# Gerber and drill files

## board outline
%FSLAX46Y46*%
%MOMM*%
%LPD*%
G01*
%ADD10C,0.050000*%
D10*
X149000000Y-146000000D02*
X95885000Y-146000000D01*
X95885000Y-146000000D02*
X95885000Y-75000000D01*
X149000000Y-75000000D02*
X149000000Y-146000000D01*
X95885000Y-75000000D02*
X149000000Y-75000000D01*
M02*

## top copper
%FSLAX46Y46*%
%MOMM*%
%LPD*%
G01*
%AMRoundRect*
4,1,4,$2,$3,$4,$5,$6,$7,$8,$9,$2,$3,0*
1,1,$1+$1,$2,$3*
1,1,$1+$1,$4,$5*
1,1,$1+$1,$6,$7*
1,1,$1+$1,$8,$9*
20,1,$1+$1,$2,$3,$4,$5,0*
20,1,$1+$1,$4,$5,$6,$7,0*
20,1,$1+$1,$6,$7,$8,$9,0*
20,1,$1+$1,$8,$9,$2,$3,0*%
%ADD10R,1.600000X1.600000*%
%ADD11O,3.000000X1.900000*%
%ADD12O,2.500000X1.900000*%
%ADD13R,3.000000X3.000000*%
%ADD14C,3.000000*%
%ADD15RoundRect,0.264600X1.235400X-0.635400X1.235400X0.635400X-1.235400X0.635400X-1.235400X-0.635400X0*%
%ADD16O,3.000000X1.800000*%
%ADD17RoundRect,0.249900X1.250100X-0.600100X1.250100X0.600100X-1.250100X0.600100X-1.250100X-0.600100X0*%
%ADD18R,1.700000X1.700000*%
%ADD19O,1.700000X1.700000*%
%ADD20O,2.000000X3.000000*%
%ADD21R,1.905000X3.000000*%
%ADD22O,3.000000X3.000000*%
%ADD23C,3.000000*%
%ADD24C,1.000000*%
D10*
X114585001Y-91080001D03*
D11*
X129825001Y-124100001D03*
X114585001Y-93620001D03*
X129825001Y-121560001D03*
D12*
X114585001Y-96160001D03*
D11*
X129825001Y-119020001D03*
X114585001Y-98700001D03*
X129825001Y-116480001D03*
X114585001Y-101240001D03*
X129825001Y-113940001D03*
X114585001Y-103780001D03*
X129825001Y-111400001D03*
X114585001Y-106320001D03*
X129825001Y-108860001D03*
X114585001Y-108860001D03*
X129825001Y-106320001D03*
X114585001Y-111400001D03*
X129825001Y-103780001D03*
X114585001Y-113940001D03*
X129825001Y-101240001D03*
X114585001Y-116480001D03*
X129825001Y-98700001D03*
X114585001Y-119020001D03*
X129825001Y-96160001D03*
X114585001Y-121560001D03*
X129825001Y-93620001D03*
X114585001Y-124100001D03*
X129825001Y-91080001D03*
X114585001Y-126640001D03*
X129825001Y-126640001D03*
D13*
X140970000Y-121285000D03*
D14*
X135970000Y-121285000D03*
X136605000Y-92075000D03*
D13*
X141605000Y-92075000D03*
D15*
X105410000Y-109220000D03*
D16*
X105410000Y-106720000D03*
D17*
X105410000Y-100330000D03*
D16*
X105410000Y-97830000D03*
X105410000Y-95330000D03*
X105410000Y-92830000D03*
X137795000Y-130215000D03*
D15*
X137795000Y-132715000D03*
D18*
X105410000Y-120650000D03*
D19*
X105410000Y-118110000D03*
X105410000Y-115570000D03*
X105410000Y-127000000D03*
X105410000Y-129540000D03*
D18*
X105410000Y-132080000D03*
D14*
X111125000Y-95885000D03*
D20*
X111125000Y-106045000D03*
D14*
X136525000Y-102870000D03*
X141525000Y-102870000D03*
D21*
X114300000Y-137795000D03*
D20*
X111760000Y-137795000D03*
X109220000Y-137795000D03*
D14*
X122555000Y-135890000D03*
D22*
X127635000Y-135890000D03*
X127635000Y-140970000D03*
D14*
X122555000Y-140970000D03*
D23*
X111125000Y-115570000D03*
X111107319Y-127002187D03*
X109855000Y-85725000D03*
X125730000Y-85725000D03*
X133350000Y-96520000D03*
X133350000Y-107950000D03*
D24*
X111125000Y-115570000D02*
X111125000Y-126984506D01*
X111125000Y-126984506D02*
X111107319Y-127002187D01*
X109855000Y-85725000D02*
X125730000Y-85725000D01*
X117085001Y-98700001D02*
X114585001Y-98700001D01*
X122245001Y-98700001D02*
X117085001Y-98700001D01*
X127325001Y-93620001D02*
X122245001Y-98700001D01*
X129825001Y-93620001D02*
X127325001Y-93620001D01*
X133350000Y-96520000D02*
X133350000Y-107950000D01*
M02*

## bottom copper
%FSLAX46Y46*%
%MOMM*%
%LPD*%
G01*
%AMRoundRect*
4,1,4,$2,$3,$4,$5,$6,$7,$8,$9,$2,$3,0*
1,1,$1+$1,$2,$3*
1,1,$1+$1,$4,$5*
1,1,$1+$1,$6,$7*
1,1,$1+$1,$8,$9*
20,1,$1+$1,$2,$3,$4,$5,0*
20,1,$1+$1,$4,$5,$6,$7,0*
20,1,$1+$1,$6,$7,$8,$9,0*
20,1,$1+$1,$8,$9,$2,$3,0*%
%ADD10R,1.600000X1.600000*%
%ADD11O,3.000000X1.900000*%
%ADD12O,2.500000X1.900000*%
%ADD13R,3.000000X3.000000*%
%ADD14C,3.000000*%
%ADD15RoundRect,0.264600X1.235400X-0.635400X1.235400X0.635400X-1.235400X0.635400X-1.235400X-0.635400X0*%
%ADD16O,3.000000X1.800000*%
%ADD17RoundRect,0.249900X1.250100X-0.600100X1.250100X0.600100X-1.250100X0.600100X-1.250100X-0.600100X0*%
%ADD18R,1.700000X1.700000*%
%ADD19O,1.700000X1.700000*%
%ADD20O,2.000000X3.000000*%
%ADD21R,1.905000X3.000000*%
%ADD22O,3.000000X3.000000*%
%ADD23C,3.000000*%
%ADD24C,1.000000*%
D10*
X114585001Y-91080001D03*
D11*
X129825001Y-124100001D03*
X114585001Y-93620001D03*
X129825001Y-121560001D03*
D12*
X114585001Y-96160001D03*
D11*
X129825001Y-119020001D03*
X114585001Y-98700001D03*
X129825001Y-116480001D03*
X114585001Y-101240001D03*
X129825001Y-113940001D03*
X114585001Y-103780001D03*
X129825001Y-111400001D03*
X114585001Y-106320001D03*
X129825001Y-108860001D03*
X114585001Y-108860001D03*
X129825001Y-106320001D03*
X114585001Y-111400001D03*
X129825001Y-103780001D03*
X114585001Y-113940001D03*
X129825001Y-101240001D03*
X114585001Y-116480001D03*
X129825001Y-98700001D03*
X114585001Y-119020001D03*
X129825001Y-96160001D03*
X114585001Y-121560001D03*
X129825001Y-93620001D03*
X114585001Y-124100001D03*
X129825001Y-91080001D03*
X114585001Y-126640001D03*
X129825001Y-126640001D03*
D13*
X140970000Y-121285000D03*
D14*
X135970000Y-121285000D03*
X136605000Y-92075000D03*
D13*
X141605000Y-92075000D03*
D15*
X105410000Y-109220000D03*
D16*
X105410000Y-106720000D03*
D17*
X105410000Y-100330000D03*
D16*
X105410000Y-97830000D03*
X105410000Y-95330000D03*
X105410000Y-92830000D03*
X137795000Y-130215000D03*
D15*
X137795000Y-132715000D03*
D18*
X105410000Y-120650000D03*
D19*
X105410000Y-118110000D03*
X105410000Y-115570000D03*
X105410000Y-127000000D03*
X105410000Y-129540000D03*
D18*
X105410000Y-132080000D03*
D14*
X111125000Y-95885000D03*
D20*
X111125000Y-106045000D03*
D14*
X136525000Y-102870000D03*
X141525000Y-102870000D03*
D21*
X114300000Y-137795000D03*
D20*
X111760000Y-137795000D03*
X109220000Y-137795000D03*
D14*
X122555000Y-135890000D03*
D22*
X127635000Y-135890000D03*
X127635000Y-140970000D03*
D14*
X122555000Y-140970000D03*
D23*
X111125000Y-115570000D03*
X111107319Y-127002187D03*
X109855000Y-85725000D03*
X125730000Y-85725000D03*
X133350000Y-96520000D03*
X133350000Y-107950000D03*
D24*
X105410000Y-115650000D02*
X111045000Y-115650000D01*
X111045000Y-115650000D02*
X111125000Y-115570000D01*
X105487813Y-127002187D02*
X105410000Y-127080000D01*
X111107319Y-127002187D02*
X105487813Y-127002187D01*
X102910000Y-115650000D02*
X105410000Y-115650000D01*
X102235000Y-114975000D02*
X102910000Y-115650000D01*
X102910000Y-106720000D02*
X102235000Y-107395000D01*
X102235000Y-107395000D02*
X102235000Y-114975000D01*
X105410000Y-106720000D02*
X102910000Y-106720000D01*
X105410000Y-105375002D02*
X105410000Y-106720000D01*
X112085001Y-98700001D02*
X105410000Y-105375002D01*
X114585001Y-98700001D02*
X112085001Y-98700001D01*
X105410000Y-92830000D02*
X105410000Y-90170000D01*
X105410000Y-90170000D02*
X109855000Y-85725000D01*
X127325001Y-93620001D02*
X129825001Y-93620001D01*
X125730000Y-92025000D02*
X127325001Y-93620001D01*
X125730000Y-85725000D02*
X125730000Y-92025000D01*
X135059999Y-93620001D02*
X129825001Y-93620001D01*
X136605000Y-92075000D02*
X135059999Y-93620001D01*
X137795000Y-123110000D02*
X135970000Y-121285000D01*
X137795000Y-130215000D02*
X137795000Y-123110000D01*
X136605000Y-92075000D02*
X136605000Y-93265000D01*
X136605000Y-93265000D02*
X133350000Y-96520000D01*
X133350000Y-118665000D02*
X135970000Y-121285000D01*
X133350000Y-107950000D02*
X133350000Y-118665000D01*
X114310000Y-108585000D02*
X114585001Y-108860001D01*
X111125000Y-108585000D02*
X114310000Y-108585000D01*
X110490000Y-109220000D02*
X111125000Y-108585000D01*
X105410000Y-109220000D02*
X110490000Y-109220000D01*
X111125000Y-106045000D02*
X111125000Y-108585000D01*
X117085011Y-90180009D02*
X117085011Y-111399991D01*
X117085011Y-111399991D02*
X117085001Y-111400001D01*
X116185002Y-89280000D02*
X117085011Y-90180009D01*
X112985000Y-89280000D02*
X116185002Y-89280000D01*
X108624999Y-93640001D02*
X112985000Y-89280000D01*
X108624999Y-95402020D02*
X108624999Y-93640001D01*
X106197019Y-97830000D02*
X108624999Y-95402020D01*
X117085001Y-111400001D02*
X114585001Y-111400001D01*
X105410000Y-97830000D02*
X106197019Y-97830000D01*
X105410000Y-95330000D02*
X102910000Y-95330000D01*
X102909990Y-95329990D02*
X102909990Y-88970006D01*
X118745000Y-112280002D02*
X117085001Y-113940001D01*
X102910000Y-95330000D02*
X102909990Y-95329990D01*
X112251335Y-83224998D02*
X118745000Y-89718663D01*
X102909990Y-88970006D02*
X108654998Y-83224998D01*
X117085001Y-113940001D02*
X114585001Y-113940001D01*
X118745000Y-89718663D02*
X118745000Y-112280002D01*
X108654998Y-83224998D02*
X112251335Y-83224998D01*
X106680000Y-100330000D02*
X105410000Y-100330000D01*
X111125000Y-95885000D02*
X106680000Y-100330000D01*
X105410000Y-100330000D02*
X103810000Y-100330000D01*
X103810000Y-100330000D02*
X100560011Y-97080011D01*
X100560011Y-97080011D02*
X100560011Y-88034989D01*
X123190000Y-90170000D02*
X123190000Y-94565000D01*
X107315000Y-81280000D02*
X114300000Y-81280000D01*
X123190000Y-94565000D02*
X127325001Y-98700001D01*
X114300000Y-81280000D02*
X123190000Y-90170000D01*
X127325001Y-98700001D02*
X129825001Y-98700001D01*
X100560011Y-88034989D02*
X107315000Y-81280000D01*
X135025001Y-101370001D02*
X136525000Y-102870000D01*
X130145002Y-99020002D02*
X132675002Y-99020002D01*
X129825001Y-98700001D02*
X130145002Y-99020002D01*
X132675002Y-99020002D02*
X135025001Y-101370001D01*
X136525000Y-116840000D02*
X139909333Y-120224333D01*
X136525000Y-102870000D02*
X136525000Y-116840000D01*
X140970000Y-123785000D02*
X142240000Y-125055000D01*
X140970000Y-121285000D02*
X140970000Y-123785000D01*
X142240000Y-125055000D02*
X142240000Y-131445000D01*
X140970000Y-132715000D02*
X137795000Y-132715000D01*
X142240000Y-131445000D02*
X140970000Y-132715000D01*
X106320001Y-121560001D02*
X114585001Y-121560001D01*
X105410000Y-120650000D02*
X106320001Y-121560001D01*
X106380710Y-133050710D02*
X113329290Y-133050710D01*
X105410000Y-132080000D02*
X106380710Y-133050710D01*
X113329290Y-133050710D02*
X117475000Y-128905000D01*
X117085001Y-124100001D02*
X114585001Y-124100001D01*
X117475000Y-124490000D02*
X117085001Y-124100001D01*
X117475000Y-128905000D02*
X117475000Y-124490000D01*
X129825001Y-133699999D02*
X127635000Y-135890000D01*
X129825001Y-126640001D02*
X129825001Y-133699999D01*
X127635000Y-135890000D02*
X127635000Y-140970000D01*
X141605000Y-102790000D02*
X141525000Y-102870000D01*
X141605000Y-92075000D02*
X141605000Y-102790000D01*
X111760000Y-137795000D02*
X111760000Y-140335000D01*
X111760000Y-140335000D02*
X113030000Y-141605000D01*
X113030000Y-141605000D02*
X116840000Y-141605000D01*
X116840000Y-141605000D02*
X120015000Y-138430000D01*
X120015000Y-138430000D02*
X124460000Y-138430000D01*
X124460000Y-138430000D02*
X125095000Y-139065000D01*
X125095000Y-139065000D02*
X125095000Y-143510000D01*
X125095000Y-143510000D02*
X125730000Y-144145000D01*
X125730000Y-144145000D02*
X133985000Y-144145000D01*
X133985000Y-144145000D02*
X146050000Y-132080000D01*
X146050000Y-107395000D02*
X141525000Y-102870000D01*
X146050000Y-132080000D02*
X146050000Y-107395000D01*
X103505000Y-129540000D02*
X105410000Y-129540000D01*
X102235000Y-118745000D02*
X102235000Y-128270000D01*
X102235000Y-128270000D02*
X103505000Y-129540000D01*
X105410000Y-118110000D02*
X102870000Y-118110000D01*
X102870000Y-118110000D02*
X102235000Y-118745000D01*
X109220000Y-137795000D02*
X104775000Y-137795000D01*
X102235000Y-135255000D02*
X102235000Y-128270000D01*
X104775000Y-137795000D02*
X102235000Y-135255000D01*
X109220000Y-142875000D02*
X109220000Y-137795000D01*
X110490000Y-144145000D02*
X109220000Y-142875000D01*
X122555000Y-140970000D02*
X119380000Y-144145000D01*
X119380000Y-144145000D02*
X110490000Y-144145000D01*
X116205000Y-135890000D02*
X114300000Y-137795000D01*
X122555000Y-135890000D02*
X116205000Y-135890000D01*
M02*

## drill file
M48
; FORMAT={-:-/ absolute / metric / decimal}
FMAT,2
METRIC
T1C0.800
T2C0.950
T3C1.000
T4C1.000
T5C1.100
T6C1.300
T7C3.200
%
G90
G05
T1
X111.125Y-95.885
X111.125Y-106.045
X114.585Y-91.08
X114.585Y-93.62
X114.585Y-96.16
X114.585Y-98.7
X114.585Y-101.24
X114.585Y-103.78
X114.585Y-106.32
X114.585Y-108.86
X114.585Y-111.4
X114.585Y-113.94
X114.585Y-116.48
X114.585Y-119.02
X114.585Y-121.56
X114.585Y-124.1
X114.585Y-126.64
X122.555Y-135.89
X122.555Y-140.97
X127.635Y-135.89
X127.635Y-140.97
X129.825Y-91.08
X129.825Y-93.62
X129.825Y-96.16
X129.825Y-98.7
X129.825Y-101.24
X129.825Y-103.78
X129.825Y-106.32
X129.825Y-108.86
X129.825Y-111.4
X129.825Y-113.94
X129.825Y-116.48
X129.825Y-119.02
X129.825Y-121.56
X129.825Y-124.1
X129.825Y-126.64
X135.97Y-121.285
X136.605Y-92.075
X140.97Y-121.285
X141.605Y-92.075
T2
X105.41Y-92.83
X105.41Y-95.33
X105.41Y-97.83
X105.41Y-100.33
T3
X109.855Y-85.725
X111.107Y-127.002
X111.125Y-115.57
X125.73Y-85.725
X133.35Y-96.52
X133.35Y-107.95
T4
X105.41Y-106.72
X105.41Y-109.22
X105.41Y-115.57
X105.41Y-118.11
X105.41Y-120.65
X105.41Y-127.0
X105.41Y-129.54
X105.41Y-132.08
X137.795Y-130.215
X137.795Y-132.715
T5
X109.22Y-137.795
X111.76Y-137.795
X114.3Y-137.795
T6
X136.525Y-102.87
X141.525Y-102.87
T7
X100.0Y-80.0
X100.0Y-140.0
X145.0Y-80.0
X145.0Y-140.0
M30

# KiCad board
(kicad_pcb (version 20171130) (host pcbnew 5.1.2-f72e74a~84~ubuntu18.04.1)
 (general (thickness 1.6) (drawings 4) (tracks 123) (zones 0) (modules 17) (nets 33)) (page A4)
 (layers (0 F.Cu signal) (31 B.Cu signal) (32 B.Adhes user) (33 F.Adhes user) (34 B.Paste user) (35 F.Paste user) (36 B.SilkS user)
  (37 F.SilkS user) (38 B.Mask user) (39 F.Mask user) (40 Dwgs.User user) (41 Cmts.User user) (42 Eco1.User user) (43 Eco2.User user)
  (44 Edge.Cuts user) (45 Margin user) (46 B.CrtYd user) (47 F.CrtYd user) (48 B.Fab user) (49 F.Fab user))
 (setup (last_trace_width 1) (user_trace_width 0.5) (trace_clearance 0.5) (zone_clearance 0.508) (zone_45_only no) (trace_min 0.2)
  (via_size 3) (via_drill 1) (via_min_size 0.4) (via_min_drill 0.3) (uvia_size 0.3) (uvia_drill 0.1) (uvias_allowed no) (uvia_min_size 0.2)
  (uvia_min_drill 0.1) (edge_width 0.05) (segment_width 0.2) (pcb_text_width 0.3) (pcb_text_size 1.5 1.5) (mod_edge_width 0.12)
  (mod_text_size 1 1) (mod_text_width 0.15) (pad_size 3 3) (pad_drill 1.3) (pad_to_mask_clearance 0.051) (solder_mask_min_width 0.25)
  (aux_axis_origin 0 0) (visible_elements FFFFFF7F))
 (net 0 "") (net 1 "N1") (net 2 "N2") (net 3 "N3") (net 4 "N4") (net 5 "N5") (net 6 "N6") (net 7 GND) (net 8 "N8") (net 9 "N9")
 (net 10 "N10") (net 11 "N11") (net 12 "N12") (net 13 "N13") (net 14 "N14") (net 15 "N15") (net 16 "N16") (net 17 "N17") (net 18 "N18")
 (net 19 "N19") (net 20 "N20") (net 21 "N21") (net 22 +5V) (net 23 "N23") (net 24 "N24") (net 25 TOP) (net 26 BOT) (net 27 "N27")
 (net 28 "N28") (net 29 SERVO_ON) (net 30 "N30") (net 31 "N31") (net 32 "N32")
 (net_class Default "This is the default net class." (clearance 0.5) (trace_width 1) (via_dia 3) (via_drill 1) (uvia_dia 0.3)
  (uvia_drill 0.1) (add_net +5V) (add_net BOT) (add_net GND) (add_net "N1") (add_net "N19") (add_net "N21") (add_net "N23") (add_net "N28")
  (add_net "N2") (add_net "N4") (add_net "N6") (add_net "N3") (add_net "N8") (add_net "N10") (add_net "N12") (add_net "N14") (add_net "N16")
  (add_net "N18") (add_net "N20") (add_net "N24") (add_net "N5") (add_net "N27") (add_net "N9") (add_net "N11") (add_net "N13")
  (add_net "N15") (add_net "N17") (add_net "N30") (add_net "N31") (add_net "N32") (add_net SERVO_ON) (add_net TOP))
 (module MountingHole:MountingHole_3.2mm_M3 (layer F.Cu) (at 145 140)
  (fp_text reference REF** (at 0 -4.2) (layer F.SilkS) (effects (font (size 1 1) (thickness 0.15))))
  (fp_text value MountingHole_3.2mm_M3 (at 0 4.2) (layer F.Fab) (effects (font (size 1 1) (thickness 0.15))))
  (pad 1 np_thru_hole circle (at 0 0) (size 3.2 3.2) (drill 3.2) (layers *.Cu *.Mask)))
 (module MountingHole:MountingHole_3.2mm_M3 (layer F.Cu) (at 100 140)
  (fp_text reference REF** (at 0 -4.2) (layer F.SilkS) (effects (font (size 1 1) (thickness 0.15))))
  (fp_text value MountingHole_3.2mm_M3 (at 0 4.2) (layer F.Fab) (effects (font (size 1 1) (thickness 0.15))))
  (pad 1 np_thru_hole circle (at 0 0) (size 3.2 3.2) (drill 3.2) (layers *.Cu *.Mask)))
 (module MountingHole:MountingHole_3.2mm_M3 (layer F.Cu) (at 100 80)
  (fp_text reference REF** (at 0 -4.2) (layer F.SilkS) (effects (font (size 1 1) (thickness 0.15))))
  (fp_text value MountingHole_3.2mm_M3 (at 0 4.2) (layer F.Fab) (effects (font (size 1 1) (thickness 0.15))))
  (pad 1 np_thru_hole circle (at 0 0) (size 3.2 3.2) (drill 3.2) (layers *.Cu *.Mask)))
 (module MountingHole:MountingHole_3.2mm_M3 (layer F.Cu) (at 145 80)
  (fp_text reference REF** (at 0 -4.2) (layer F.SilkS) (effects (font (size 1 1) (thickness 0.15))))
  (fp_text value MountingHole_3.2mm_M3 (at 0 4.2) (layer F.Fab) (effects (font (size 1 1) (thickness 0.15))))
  (pad 1 np_thru_hole circle (at 0 0) (size 3.2 3.2) (drill 3.2) (layers *.Cu *.Mask)))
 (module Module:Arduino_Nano (layer F.Cu) (at 114.585001 91.080001)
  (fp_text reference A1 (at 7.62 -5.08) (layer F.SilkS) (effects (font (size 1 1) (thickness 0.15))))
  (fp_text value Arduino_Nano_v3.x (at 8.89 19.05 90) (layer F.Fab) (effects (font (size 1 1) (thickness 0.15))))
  (pad 1 thru_hole rect (at 0 0) (size 1.6 1.6) (drill 0.8) (layers *.Cu *.Mask) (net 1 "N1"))
  (pad 17 thru_hole oval (at 15.24 33.02) (size 3 1.9) (drill 0.8) (layers *.Cu *.Mask) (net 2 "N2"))
  (pad 2 thru_hole oval (at 0 2.54) (size 3 1.9) (drill 0.8) (layers *.Cu *.Mask) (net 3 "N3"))
  (pad 18 thru_hole oval (at 15.24 30.48) (size 3 1.9) (drill 0.8) (layers *.Cu *.Mask) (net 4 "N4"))
  (pad 3 thru_hole oval (at 0 5.08) (size 2.5 1.9) (drill 0.8) (layers *.Cu *.Mask) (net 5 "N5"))
  (pad 19 thru_hole oval (at 15.24 27.94) (size 3 1.9) (drill 0.8) (layers *.Cu *.Mask) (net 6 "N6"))
  (pad 4 thru_hole oval (at 0 7.62) (size 3 1.9) (drill 0.8) (layers *.Cu *.Mask) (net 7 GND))
  (pad 20 thru_hole oval (at 15.24 25.4) (size 3 1.9) (drill 0.8) (layers *.Cu *.Mask) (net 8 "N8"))
  (pad 5 thru_hole oval (at 0 10.16) (size 3 1.9) (drill 0.8) (layers *.Cu *.Mask) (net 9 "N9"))
  (pad 21 thru_hole oval (at 15.24 22.86) (size 3 1.9) (drill 0.8) (layers *.Cu *.Mask) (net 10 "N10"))
  (pad 6 thru_hole oval (at 0 12.7) (size 3 1.9) (drill 0.8) (layers *.Cu *.Mask) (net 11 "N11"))
  (pad 22 thru_hole oval (at 15.24 20.32) (size 3 1.9) (drill 0.8) (layers *.Cu *.Mask) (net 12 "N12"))
  (pad 7 thru_hole oval (at 0 15.24) (size 3 1.9) (drill 0.8) (layers *.Cu *.Mask) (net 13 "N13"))
  (pad 23 thru_hole oval (at 15.24 17.78) (size 3 1.9) (drill 0.8) (layers *.Cu *.Mask) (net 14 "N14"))
  (pad 8 thru_hole oval (at 0 17.78) (size 3 1.9) (drill 0.8) (layers *.Cu *.Mask) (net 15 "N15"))
  (pad 24 thru_hole oval (at 15.24 15.24) (size 3 1.9) (drill 0.8) (layers *.Cu *.Mask) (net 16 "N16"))
  (pad 9 thru_hole oval (at 0 20.32) (size 3 1.9) (drill 0.8) (layers *.Cu *.Mask) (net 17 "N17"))
  (pad 25 thru_hole oval (at 15.24 12.7) (size 3 1.9) (drill 0.8) (layers *.Cu *.Mask) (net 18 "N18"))
  (pad 10 thru_hole oval (at 0 22.86) (size 3 1.9) (drill 0.8) (layers *.Cu *.Mask) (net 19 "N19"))
  (pad 26 thru_hole oval (at 15.24 10.16) (size 3 1.9) (drill 0.8) (layers *.Cu *.Mask) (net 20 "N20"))
  (pad 11 thru_hole oval (at 0 25.4) (size 3 1.9) (drill 0.8) (layers *.Cu *.Mask) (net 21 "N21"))
  (pad 27 thru_hole oval (at 15.24 7.62) (size 3 1.9) (drill 0.8) (layers *.Cu *.Mask) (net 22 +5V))
  (pad 12 thru_hole oval (at 0 27.94) (size 3 1.9) (drill 0.8) (layers *.Cu *.Mask) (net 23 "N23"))
  (pad 28 thru_hole oval (at 15.24 5.08) (size 3 1.9) (drill 0.8) (layers *.Cu *.Mask) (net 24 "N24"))
  (pad 13 thru_hole oval (at 0 30.48) (size 3 1.9) (drill 0.8) (layers *.Cu *.Mask) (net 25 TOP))
  (pad 29 thru_hole oval (at 15.24 2.54) (size 3 1.9) (drill 0.8) (layers *.Cu *.Mask) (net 7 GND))
  (pad 14 thru_hole oval (at 0 33.02) (size 3 1.9) (drill 0.8) (layers *.Cu *.Mask) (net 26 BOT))
  (pad 30 thru_hole oval (at 15.24 0) (size 3 1.9) (drill 0.8) (layers *.Cu *.Mask) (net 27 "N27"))
  (pad 15 thru_hole oval (at 0 35.56) (size 3 1.9) (drill 0.8) (layers *.Cu *.Mask) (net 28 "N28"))
  (pad 16 thru_hole oval (at 15.24 35.56) (size 3 1.9) (drill 0.8) (layers *.Cu *.Mask) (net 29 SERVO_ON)))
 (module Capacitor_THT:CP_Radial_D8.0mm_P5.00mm (layer F.Cu) (at 140.97 121.285 180)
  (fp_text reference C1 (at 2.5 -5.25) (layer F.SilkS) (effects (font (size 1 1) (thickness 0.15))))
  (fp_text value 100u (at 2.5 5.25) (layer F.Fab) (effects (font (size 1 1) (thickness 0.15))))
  (pad 1 thru_hole rect (at 0 0 180) (size 3 3) (drill 0.8) (layers *.Cu *.Mask) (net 22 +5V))
  (pad 2 thru_hole circle (at 5 0 180) (size 3 3) (drill 0.8) (layers *.Cu *.Mask) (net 7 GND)))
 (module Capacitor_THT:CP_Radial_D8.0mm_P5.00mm (layer F.Cu) (at 141.605 92.075 180)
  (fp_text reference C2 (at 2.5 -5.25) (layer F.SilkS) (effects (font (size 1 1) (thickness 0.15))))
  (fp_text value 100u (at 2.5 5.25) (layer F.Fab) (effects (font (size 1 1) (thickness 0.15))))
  (pad 2 thru_hole circle (at 5 0 180) (size 3 3) (drill 0.8) (layers *.Cu *.Mask) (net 7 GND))
  (pad 1 thru_hole rect (at 0 0 180) (size 3 3) (drill 0.8) (layers *.Cu *.Mask) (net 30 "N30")))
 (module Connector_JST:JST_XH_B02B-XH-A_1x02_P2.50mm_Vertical (layer F.Cu) (at 105.41 109.22 90)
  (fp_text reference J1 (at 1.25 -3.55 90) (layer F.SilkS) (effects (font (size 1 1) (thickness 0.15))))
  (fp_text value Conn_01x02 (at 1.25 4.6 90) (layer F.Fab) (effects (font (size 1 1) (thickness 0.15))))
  (pad 1 thru_hole roundrect (at 0 0 90) (size 1.8 3) (drill 1) (layers *.Cu *.Mask) (roundrect_rratio 0.147) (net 15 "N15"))
  (pad 2 thru_hole oval (at 2.5 0 90) (size 1.8 3) (drill 1) (layers *.Cu *.Mask) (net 7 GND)))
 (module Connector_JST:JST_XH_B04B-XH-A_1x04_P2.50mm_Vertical (layer F.Cu) (at 105.41 100.33 90)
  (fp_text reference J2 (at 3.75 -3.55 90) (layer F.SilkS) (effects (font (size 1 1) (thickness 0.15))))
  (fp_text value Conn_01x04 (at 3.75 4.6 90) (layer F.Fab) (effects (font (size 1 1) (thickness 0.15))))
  (pad 1 thru_hole roundrect (at 0 0 90) (size 1.7 3) (drill 0.95) (layers *.Cu *.Mask) (roundrect_rratio 0.147) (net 22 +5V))
  (pad 2 thru_hole oval (at 2.5 0 90) (size 1.8 3) (drill 0.95) (layers *.Cu *.Mask) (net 17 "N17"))
  (pad 3 thru_hole oval (at 5 0 90) (size 1.8 3) (drill 0.95) (layers *.Cu *.Mask) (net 19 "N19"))
  (pad 4 thru_hole oval (at 7.5 0 90) (size 1.8 3) (drill 0.95) (layers *.Cu *.Mask) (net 7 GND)))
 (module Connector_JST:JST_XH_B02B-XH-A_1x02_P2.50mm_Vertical (layer F.Cu) (at 137.795 132.715 90)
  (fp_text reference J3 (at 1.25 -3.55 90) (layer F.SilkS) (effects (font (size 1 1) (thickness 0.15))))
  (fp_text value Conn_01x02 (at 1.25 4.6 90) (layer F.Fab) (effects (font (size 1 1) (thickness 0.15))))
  (pad 2 thru_hole oval (at 2.5 0 90) (size 1.8 3) (drill 1) (layers *.Cu *.Mask) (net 7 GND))
  (pad 1 thru_hole roundrect (at 0 0 90) (size 1.8 3) (drill 1) (layers *.Cu *.Mask) (roundrect_rratio 0.147) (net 22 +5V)))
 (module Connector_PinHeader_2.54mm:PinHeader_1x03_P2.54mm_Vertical (layer F.Cu) (at 105.41 120.65 180)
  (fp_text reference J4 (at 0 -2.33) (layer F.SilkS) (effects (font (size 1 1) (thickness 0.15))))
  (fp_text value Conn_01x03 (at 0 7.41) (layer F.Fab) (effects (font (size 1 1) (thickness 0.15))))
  (pad 1 thru_hole rect (at 0 0 180) (size 1.7 1.7) (drill 1) (layers *.Cu *.Mask) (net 25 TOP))
  (pad 2 thru_hole oval (at 0 2.54 180) (size 1.7 1.7) (drill 1) (layers *.Cu *.Mask) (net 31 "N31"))
  (pad 3 thru_hole oval (at 0 5.08 180) (size 1.7 1.7) (drill 1) (layers *.Cu *.Mask) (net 7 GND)))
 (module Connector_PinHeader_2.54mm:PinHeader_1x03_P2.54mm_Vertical (layer F.Cu) (at 105.41 132.08 180)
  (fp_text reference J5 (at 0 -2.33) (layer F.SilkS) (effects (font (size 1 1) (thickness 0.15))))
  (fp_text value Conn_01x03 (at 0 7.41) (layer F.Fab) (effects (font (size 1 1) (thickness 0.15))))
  (pad 3 thru_hole oval (at 0 5.08 180) (size 1.7 1.7) (drill 1) (layers *.Cu *.Mask) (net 7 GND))
  (pad 2 thru_hole oval (at 0 2.54 180) (size 1.7 1.7) (drill 1) (layers *.Cu *.Mask) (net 31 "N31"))
  (pad 1 thru_hole rect (at 0 0 180) (size 1.7 1.7) (drill 1) (layers *.Cu *.Mask) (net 26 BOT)))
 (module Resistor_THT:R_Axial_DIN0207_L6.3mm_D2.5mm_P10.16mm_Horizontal (layer F.Cu) (at 111.125 95.885 270)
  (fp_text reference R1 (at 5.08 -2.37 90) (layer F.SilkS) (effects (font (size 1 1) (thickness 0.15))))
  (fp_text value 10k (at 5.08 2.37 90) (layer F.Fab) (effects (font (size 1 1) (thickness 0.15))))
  (pad 1 thru_hole circle (at 0 0 270) (size 3 3) (drill 0.8) (layers *.Cu *.Mask) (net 22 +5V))
  (pad 2 thru_hole oval (at 10.16 0 270) (size 3 2) (drill 0.8) (layers *.Cu *.Mask) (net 15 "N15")))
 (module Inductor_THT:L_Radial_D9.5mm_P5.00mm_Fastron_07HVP (layer F.Cu) (at 136.525 102.87)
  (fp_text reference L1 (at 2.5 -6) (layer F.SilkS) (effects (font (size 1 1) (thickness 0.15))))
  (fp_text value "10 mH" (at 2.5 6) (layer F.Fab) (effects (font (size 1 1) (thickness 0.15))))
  (pad 1 thru_hole circle (at 0 0) (size 3 3) (drill 1.3) (layers *.Cu *.Mask) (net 22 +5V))
  (pad 2 thru_hole circle (at 5 0) (size 3 3) (drill 1.3) (layers *.Cu *.Mask) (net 30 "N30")))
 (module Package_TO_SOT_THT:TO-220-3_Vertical (layer F.Cu) (at 114.3 137.795 180)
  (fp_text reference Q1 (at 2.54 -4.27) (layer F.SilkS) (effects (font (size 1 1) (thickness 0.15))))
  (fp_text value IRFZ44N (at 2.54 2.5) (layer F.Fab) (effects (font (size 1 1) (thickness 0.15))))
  (pad 1 thru_hole rect (at 0 0 180) (size 1.905 3) (drill 1.1) (layers *.Cu *.Mask) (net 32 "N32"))
  (pad 2 thru_hole oval (at 2.54 0 180) (size 2 3) (drill 1.1) (layers *.Cu *.Mask) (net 30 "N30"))
  (pad 3 thru_hole oval (at 5.08 0 180) (size 2 3) (drill 1.1) (layers *.Cu *.Mask) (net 31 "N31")))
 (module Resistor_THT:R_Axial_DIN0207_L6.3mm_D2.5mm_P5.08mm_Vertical (layer F.Cu) (at 122.555 135.89)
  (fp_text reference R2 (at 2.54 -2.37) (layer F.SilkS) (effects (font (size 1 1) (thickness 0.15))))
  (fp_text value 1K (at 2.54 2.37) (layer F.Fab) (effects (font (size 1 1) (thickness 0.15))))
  (pad 1 thru_hole circle (at 0 0) (size 3 3) (drill 0.8) (layers *.Cu *.Mask) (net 32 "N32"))
  (pad 2 thru_hole oval (at 5.08 0) (size 3 3) (drill 0.8) (layers *.Cu *.Mask) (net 29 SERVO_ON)))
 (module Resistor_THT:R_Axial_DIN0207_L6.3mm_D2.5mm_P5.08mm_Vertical (layer F.Cu) (at 122.555 140.97)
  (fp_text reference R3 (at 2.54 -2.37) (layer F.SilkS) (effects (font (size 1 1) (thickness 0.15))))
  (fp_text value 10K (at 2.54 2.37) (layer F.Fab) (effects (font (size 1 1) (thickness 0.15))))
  (pad 2 thru_hole oval (at 5.08 0) (size 3 3) (drill 0.8) (layers *.Cu *.Mask) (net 29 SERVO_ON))
  (pad 1 thru_hole circle (at 0 0) (size 3 3) (drill 0.8) (layers *.Cu *.Mask) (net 31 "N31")))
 (gr_line (start 149 146) (end 95.885 146) (layer Edge.Cuts) (width 0.05))
 (gr_line (start 95.885 146) (end 95.885 75) (layer Edge.Cuts) (width 0.05))
 (gr_line (start 149 75) (end 149 146) (layer Edge.Cuts) (width 0.05))
 (gr_line (start 95.885 75) (end 149 75) (layer Edge.Cuts) (width 0.05))
 (segment (start 105.41 115.65) (end 111.045 115.65) (width 1) (layer B.Cu) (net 7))
 (via (at 111.125 115.57) (size 3) (drill 1) (layers F.Cu B.Cu) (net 7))
 (segment (start 111.045 115.65) (end 111.125 115.57) (width 1) (layer B.Cu) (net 7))
 (via (at 111.107319 127.002187) (size 3) (drill 1) (layers F.Cu B.Cu) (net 7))
 (segment (start 111.125 115.57) (end 111.125 126.984506) (width 1) (layer F.Cu) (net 7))
 (segment (start 111.125 126.984506) (end 111.107319 127.002187) (width 1) (layer F.Cu) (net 7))
 (segment (start 105.487813 127.002187) (end 105.41 127.08) (width 1) (layer B.Cu) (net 7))
 (segment (start 111.107319 127.002187) (end 105.487813 127.002187) (width 1) (layer B.Cu) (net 7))
 (segment (start 102.91 115.65) (end 105.41 115.65) (width 1) (layer B.Cu) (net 7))
 (segment (start 102.235 114.975) (end 102.91 115.65) (width 1) (layer B.Cu) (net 7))
 (segment (start 102.91 106.72) (end 102.235 107.395) (width 1) (layer B.Cu) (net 7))
 (segment (start 102.235 107.395) (end 102.235 114.975) (width 1) (layer B.Cu) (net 7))
 (segment (start 105.41 106.72) (end 102.91 106.72) (width 1) (layer B.Cu) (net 7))
 (segment (start 105.41 105.375002) (end 105.41 106.72) (width 1) (layer B.Cu) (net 7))
 (segment (start 112.085001 98.700001) (end 105.41 105.375002) (width 1) (layer B.Cu) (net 7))
 (segment (start 114.585001 98.700001) (end 112.085001 98.700001) (width 1) (layer B.Cu) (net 7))
 (segment (start 105.41 92.83) (end 105.41 90.17) (width 1) (layer B.Cu) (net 7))
 (segment (start 105.41 90.17) (end 109.855 85.725) (width 1) (layer B.Cu) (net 7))
 (via (at 109.855 85.725) (size 3) (drill 1) (layers F.Cu B.Cu) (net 7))
 (via (at 125.73 85.725) (size 3) (drill 1) (layers F.Cu B.Cu) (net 7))
 (segment (start 109.855 85.725) (end 125.73 85.725) (width 1) (layer F.Cu) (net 7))
 (segment (start 127.325001 93.620001) (end 129.825001 93.620001) (width 1) (layer B.Cu) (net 7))
 (segment (start 125.73 92.025) (end 127.325001 93.620001) (width 1) (layer B.Cu) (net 7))
 (segment (start 125.73 85.725) (end 125.73 92.025) (width 1) (layer B.Cu) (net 7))
 (segment (start 117.085001 98.700001) (end 114.585001 98.700001) (width 1) (layer F.Cu) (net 7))
 (segment (start 122.245001 98.700001) (end 117.085001 98.700001) (width 1) (layer F.Cu) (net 7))
 (segment (start 127.325001 93.620001) (end 122.245001 98.700001) (width 1) (layer F.Cu) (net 7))
 (segment (start 129.825001 93.620001) (end 127.325001 93.620001) (width 1) (layer F.Cu) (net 7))
 (segment (start 135.059999 93.620001) (end 129.825001 93.620001) (width 1) (layer B.Cu) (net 7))
 (segment (start 136.605 92.075) (end 135.059999 93.620001) (width 1) (layer B.Cu) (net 7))
 (segment (start 137.795 123.11) (end 135.97 121.285) (width 1) (layer B.Cu) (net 7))
 (segment (start 137.795 130.215) (end 137.795 123.11) (width 1) (layer B.Cu) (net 7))
 (via (at 133.35 96.52) (size 3) (drill 1) (layers F.Cu B.Cu) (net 7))
 (segment (start 136.605 92.075) (end 136.605 93.265) (width 1) (layer B.Cu) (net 7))
 (segment (start 136.605 93.265) (end 133.35 96.52) (width 1) (layer B.Cu) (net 7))
 (via (at 133.35 107.95) (size 3) (drill 1) (layers F.Cu B.Cu) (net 7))
 (segment (start 133.35 96.52) (end 133.35 107.95) (width 1) (layer F.Cu) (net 7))
 (segment (start 133.35 118.665) (end 135.97 121.285) (width 1) (layer B.Cu) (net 7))
 (segment (start 133.35 107.95) (end 133.35 118.665) (width 1) (layer B.Cu) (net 7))
 (segment (start 114.31 108.585) (end 114.585001 108.860001) (width 1) (layer B.Cu) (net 15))
 (segment (start 111.125 108.585) (end 114.31 108.585) (width 1) (layer B.Cu) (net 15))
 (segment (start 110.49 109.22) (end 111.125 108.585) (width 1) (layer B.Cu) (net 15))
 (segment (start 105.41 109.22) (end 110.49 109.22) (width 1) (layer B.Cu) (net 15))
 (segment (start 111.125 106.045) (end 111.125 108.585) (width 1) (layer B.Cu) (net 15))
 (segment (start 117.085011 90.180009) (end 117.085011 111.399991) (width 1) (layer B.Cu) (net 17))
 (segment (start 117.085011 111.399991) (end 117.085001 111.400001) (width 1) (layer B.Cu) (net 17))
 (segment (start 116.185002 89.28) (end 117.085011 90.180009) (width 1) (layer B.Cu) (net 17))
 (segment (start 112.985 89.28) (end 116.185002 89.28) (width 1) (layer B.Cu) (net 17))
 (segment (start 108.624999 93.640001) (end 112.985 89.28) (width 1) (layer B.Cu) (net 17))
 (segment (start 108.624999 95.40202) (end 108.624999 93.640001) (width 1) (layer B.Cu) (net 17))
 (segment (start 106.197019 97.83) (end 108.624999 95.40202) (width 1) (layer B.Cu) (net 17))
 (segment (start 117.085001 111.400001) (end 114.585001 111.400001) (width 1) (layer B.Cu) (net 17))
 (segment (start 105.41 97.83) (end 106.197019 97.83) (width 1) (layer B.Cu) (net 17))
 (segment (start 105.41 95.33) (end 102.91 95.33) (width 1) (layer B.Cu) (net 19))
 (segment (start 102.90999 95.32999) (end 102.90999 88.970006) (width 1) (layer B.Cu) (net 19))
 (segment (start 118.745 112.280002) (end 117.085001 113.940001) (width 1) (layer B.Cu) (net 19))
 (segment (start 102.91 95.33) (end 102.90999 95.32999) (width 1) (layer B.Cu) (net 19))
 (segment (start 112.251335 83.224998) (end 118.745 89.718663) (width 1) (layer B.Cu) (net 19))
 (segment (start 102.90999 88.970006) (end 108.654998 83.224998) (width 1) (layer B.Cu) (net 19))
 (segment (start 117.085001 113.940001) (end 114.585001 113.940001) (width 1) (layer B.Cu) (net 19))
 (segment (start 118.745 89.718663) (end 118.745 112.280002) (width 1) (layer B.Cu) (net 19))
 (segment (start 108.654998 83.224998) (end 112.251335 83.224998) (width 1) (layer B.Cu) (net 19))
 (segment (start 106.68 100.33) (end 105.41 100.33) (width 1) (layer B.Cu) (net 22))
 (segment (start 111.125 95.885) (end 106.68 100.33) (width 1) (layer B.Cu) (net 22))
 (segment (start 105.41 100.33) (end 103.81 100.33) (width 1) (layer B.Cu) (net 22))
 (segment (start 103.81 100.33) (end 100.560011 97.080011) (width 1) (layer B.Cu) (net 22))
 (segment (start 100.560011 97.080011) (end 100.560011 88.034989) (width 1) (layer B.Cu) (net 22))
 (segment (start 123.19 90.17) (end 123.19 94.565) (width 1) (layer B.Cu) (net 22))
 (segment (start 107.315 81.28) (end 114.3 81.28) (width 1) (layer B.Cu) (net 22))
 (segment (start 123.19 94.565) (end 127.325001 98.700001) (width 1) (layer B.Cu) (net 22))
 (segment (start 114.3 81.28) (end 123.19 90.17) (width 1) (layer B.Cu) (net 22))
 (segment (start 127.325001 98.700001) (end 129.825001 98.700001) (width 1) (layer B.Cu) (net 22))
 (segment (start 100.560011 88.034989) (end 107.315 81.28) (width 1) (layer B.Cu) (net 22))
 (segment (start 135.025001 101.370001) (end 136.525 102.87) (width 1) (layer B.Cu) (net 22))
 (segment (start 130.145002 99.020002) (end 132.675002 99.020002) (width 1) (layer B.Cu) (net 22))
 (segment (start 129.825001 98.700001) (end 130.145002 99.020002) (width 1) (layer B.Cu) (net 22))
 (segment (start 132.675002 99.020002) (end 135.025001 101.370001) (width 1) (layer B.Cu) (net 22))
 (segment (start 136.525 116.84) (end 139.909333 120.224333) (width 1) (layer B.Cu) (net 22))
 (segment (start 136.525 102.87) (end 136.525 116.84) (width 1) (layer B.Cu) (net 22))
 (segment (start 140.97 123.785) (end 142.24 125.055) (width 1) (layer B.Cu) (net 22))
 (segment (start 140.97 121.285) (end 140.97 123.785) (width 1) (layer B.Cu) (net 22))
 (segment (start 142.24 125.055) (end 142.24 131.445) (width 1) (layer B.Cu) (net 22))
 (segment (start 140.97 132.715) (end 137.795 132.715) (width 1) (layer B.Cu) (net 22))
 (segment (start 142.24 131.445) (end 140.97 132.715) (width 1) (layer B.Cu) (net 22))
 (segment (start 106.320001 121.560001) (end 114.585001 121.560001) (width 1) (layer B.Cu) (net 25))
 (segment (start 105.41 120.65) (end 106.320001 121.560001) (width 1) (layer B.Cu) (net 25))
 (segment (start 106.38071 133.05071) (end 113.32929 133.05071) (width 1) (layer B.Cu) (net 26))
 (segment (start 105.41 132.08) (end 106.38071 133.05071) (width 1) (layer B.Cu) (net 26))
 (segment (start 113.32929 133.05071) (end 117.475 128.905) (width 1) (layer B.Cu) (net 26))
 (segment (start 117.085001 124.100001) (end 114.585001 124.100001) (width 1) (layer B.Cu) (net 26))
 (segment (start 117.475 124.49) (end 117.085001 124.100001) (width 1) (layer B.Cu) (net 26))
 (segment (start 117.475 128.905) (end 117.475 124.49) (width 1) (layer B.Cu) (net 26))
 (segment (start 129.825001 133.699999) (end 127.635 135.89) (width 1) (layer B.Cu) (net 29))
 (segment (start 129.825001 126.640001) (end 129.825001 133.699999) (width 1) (layer B.Cu) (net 29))
 (segment (start 127.635 135.89) (end 127.635 140.97) (width 1) (layer B.Cu) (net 29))
 (segment (start 141.605 102.79) (end 141.525 102.87) (width 1) (layer B.Cu) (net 30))
 (segment (start 141.605 92.075) (end 141.605 102.79) (width 1) (layer B.Cu) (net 30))
 (segment (start 111.76 137.795) (end 111.76 140.335) (width 1) (layer B.Cu) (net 30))
 (segment (start 111.76 140.335) (end 113.03 141.605) (width 1) (layer B.Cu) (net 30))
 (segment (start 113.03 141.605) (end 116.84 141.605) (width 1) (layer B.Cu) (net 30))
 (segment (start 116.84 141.605) (end 120.015 138.43) (width 1) (layer B.Cu) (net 30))
 (segment (start 120.015 138.43) (end 124.46 138.43) (width 1) (layer B.Cu) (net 30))
 (segment (start 124.46 138.43) (end 125.095 139.065) (width 1) (layer B.Cu) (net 30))
 (segment (start 125.095 139.065) (end 125.095 143.51) (width 1) (layer B.Cu) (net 30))
 (segment (start 125.095 143.51) (end 125.73 144.145) (width 1) (layer B.Cu) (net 30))
 (segment (start 125.73 144.145) (end 133.985 144.145) (width 1) (layer B.Cu) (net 30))
 (segment (start 133.985 144.145) (end 146.05 132.08) (width 1) (layer B.Cu) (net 30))
 (segment (start 146.05 107.395) (end 141.525 102.87) (width 1) (layer B.Cu) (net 30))
 (segment (start 146.05 132.08) (end 146.05 107.395) (width 1) (layer B.Cu) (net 30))
 (segment (start 103.505 129.54) (end 105.41 129.54) (width 1) (layer B.Cu) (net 31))
 (segment (start 102.235 118.745) (end 102.235 128.27) (width 1) (layer B.Cu) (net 31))
 (segment (start 102.235 128.27) (end 103.505 129.54) (width 1) (layer B.Cu) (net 31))
 (segment (start 105.41 118.11) (end 102.87 118.11) (width 1) (layer B.Cu) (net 31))
 (segment (start 102.87 118.11) (end 102.235 118.745) (width 1) (layer B.Cu) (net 31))
 (segment (start 109.22 137.795) (end 104.775 137.795) (width 1) (layer B.Cu) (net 31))
 (segment (start 102.235 135.255) (end 102.235 128.27) (width 1) (layer B.Cu) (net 31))
 (segment (start 104.775 137.795) (end 102.235 135.255) (width 1) (layer B.Cu) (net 31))
 (segment (start 109.22 142.875) (end 109.22 137.795) (width 1) (layer B.Cu) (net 31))
 (segment (start 110.49 144.145) (end 109.22 142.875) (width 1) (layer B.Cu) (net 31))
 (segment (start 122.555 140.97) (end 119.38 144.145) (width 1) (layer B.Cu) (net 31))
 (segment (start 119.38 144.145) (end 110.49 144.145) (width 1) (layer B.Cu) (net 31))
 (segment (start 116.205 135.89) (end 114.3 137.795) (width 1) (layer B.Cu) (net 32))
 (segment (start 122.555 135.89) (end 116.205 135.89) (width 1) (layer B.Cu) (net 32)))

